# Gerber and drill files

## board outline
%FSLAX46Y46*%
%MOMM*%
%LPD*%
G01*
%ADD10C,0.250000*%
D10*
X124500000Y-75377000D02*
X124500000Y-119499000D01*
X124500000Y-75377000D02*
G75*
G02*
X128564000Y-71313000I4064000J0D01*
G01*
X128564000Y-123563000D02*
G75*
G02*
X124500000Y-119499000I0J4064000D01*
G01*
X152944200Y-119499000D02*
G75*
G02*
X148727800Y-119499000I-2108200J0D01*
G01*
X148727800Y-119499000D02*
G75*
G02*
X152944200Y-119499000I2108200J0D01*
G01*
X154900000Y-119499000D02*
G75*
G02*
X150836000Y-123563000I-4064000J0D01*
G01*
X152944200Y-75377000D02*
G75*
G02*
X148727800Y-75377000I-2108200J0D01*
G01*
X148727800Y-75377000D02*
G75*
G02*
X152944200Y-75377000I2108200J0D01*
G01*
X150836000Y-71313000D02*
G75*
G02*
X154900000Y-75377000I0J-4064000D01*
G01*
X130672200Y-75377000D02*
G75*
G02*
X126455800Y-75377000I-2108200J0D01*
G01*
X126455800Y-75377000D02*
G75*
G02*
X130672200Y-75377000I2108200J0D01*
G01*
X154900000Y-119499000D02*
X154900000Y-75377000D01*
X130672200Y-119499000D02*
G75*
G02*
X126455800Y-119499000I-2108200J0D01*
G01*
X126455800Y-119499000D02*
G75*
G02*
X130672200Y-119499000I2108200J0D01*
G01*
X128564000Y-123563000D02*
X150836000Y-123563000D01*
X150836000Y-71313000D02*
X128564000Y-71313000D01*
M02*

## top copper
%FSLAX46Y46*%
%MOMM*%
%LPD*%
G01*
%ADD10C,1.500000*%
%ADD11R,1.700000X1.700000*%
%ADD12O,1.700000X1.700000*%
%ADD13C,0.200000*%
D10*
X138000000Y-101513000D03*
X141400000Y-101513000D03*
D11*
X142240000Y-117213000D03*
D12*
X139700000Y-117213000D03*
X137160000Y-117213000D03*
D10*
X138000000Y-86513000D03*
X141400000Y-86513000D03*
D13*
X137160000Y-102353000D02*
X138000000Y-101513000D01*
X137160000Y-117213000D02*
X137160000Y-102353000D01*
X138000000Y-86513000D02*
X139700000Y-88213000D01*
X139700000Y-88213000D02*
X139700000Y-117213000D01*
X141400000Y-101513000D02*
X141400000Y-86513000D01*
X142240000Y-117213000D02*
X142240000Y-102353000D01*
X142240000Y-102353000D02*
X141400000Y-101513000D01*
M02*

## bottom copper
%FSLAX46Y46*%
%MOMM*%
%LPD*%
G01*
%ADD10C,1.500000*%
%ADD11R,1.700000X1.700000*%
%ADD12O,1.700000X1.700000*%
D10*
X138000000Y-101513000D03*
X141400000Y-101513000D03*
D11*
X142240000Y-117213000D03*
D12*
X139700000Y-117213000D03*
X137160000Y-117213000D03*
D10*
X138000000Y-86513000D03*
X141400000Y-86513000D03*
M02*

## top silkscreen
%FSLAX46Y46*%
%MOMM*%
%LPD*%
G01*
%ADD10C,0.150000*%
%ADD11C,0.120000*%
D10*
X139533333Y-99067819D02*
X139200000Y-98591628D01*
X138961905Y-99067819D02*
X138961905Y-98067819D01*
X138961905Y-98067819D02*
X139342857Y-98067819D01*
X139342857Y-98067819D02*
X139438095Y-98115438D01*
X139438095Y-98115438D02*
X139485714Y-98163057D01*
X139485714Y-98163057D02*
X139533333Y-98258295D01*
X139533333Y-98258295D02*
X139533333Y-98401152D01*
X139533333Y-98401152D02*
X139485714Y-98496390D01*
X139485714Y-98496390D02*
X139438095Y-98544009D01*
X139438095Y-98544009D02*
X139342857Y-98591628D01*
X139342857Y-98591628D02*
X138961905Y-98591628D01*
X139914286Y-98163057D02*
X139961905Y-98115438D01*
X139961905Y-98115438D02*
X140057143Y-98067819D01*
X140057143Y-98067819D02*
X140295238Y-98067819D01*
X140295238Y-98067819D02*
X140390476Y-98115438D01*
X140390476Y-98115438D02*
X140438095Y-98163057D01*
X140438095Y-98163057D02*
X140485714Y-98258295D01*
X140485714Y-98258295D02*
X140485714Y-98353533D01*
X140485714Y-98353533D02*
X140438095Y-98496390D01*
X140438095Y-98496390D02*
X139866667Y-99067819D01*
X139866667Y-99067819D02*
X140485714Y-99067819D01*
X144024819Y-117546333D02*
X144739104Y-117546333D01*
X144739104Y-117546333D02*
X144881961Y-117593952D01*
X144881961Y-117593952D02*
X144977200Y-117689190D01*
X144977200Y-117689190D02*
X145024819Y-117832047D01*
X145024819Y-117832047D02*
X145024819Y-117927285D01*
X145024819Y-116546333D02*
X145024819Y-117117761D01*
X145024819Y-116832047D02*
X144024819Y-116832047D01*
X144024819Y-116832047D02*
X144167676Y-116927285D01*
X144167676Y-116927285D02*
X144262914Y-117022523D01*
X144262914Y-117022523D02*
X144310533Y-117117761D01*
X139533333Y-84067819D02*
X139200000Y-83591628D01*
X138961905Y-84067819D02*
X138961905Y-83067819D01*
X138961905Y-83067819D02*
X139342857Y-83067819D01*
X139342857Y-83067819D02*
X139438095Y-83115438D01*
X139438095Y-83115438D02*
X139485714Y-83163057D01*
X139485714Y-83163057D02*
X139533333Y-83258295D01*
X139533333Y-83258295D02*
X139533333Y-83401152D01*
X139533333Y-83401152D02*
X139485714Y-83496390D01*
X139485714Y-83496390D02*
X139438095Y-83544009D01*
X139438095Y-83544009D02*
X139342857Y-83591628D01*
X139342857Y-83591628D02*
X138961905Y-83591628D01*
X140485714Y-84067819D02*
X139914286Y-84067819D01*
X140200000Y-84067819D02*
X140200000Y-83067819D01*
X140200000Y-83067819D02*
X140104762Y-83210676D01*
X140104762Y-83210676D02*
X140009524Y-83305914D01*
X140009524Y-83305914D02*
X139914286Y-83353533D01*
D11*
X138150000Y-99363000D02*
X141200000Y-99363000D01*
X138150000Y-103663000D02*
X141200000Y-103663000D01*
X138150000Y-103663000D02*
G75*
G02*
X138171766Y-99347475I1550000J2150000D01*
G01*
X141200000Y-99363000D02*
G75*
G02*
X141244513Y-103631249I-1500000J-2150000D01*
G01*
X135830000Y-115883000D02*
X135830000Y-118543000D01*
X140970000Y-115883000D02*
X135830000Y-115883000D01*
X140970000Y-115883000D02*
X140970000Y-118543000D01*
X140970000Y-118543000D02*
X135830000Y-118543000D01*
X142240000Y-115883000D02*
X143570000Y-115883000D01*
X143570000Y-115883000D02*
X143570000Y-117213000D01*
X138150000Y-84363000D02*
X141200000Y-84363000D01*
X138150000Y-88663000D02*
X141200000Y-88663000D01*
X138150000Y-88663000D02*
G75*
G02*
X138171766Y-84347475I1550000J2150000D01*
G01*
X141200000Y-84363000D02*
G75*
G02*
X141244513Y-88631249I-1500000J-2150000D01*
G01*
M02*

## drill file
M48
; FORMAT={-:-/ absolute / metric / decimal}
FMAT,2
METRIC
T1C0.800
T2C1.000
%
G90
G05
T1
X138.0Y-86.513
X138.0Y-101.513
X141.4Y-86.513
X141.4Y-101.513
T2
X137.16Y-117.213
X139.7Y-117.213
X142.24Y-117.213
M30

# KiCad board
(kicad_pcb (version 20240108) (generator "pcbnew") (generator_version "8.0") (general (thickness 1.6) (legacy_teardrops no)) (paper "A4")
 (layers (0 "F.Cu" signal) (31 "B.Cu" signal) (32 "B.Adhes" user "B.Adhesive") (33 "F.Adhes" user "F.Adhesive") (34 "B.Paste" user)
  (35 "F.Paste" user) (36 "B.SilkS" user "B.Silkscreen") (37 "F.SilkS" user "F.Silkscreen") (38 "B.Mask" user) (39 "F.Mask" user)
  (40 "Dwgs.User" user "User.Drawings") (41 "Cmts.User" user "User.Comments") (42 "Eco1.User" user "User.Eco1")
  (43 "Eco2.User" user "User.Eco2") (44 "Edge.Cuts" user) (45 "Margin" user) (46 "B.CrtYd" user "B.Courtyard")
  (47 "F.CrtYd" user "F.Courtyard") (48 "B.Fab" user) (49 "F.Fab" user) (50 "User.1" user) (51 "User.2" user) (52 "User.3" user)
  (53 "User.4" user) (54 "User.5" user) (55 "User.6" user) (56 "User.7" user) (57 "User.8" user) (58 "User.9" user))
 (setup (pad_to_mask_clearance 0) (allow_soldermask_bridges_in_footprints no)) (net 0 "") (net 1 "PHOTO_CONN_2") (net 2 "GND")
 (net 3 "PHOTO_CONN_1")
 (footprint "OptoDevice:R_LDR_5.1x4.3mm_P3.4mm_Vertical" (layer "F.Cu") (at 138 101.513)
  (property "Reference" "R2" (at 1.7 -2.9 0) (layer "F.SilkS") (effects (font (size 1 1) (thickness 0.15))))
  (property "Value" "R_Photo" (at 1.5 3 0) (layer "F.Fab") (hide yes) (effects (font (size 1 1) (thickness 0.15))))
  (fp_line (start 0.15 -2.15) (end 3.2 -2.15) (stroke (width 0.12) (type solid)) (layer "F.SilkS"))
  (fp_line (start 0.15 2.15) (end 3.2 2.15) (stroke (width 0.12) (type solid)) (layer "F.SilkS"))
  (fp_arc (start 0.15 2.15) (mid -0.950438 -0.013368) (end 0.171766 -2.165525) (stroke (width 0.12) (type solid)) (layer "F.SilkS"))
  (fp_arc (start 3.2 -2.15) (mid 4.321403 -0.027338) (end 3.244513 2.118249) (stroke (width 0.12) (type solid)) (layer "F.SilkS"))
  (pad "1" thru_hole circle (at 0 0) (size 1.5 1.5) (drill 0.8) (layers "*.Cu" "*.Mask") (remove_unused_layers no) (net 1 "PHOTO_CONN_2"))
  (pad "2" thru_hole circle (at 3.4 0) (size 1.5 1.5) (drill 0.8) (layers "*.Cu" "*.Mask") (remove_unused_layers no) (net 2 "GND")))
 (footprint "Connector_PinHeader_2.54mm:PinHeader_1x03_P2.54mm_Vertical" (layer "F.Cu") (at 142.24 117.213 -90)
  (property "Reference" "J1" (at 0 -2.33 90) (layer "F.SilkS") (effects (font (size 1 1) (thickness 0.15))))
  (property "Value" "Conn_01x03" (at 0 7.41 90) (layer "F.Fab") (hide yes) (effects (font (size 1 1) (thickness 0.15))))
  (fp_line (start -1.33 6.41) (end 1.33 6.41) (stroke (width 0.12) (type solid)) (layer "F.SilkS"))
  (fp_line (start -1.33 1.27) (end -1.33 6.41) (stroke (width 0.12) (type solid)) (layer "F.SilkS"))
  (fp_line (start -1.33 1.27) (end 1.33 1.27) (stroke (width 0.12) (type solid)) (layer "F.SilkS"))
  (fp_line (start 1.33 1.27) (end 1.33 6.41) (stroke (width 0.12) (type solid)) (layer "F.SilkS"))
  (fp_line (start -1.33 0) (end -1.33 -1.33) (stroke (width 0.12) (type solid)) (layer "F.SilkS"))
  (fp_line (start -1.33 -1.33) (end 0 -1.33) (stroke (width 0.12) (type solid)) (layer "F.SilkS"))
  (pad "1" thru_hole rect (at 0 0 270) (size 1.7 1.7) (drill 1) (layers "*.Cu" "*.Mask") (remove_unused_layers no) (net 2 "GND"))
  (pad "2" thru_hole oval (at 0 2.54 270) (size 1.7 1.7) (drill 1) (layers "*.Cu" "*.Mask") (remove_unused_layers no) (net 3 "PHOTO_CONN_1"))
  (pad "3" thru_hole oval (at 0 5.08 270) (size 1.7 1.7) (drill 1) (layers "*.Cu" "*.Mask") (remove_unused_layers no) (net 1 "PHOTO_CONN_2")))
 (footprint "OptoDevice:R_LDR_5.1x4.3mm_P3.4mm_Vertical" (layer "F.Cu") (at 138 86.513)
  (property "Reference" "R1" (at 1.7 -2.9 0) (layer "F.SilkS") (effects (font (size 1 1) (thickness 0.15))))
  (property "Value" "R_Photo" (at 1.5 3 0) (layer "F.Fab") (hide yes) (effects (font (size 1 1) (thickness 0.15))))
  (fp_line (start 0.15 -2.15) (end 3.2 -2.15) (stroke (width 0.12) (type solid)) (layer "F.SilkS"))
  (fp_line (start 0.15 2.15) (end 3.2 2.15) (stroke (width 0.12) (type solid)) (layer "F.SilkS"))
  (fp_arc (start 0.15 2.15) (mid -0.950438 -0.013368) (end 0.171766 -2.165525) (stroke (width 0.12) (type solid)) (layer "F.SilkS"))
  (fp_arc (start 3.2 -2.15) (mid 4.321403 -0.027338) (end 3.244513 2.118249) (stroke (width 0.12) (type solid)) (layer "F.SilkS"))
  (pad "1" thru_hole circle (at 0 0) (size 1.5 1.5) (drill 0.8) (layers "*.Cu" "*.Mask") (remove_unused_layers no) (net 3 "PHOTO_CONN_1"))
  (pad "2" thru_hole circle (at 3.4 0) (size 1.5 1.5) (drill 0.8) (layers "*.Cu" "*.Mask") (remove_unused_layers no) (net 2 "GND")))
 (gr_line (start 124.5 75.377) (end 124.5 119.499) (locked yes) (stroke (width 0.25) (type default)) (layer "Edge.Cuts"))
 (gr_arc (start 124.5 75.377) (mid 125.690318 72.503318) (end 128.564 71.313) (locked yes) (stroke (width 0.25) (type default))
  (layer "Edge.Cuts"))
 (gr_arc (start 128.564 123.563) (mid 125.690318 122.372682) (end 124.5 119.499) (locked yes) (stroke (width 0.25) (type default))
  (layer "Edge.Cuts"))
 (gr_circle (center 150.836 119.499) (end 152.9442 119.499) (locked yes) (stroke (width 0.25) (type default)) (fill none)
  (layer "Edge.Cuts"))
 (gr_arc (start 154.9 119.499) (mid 153.709682 122.372682) (end 150.836 123.563) (locked yes) (stroke (width 0.25) (type default))
  (layer "Edge.Cuts"))
 (gr_circle (center 150.836 75.377) (end 152.9442 75.377) (locked yes) (stroke (width 0.25) (type default)) (fill none) (layer "Edge.Cuts"))
 (gr_arc (start 150.836 71.313) (mid 153.709682 72.503318) (end 154.9 75.377) (locked yes) (stroke (width 0.25) (type default))
  (layer "Edge.Cuts"))
 (gr_circle (center 128.564 75.377) (end 130.6722 75.377) (locked yes) (stroke (width 0.25) (type default)) (fill none) (layer "Edge.Cuts"))
 (gr_line (start 154.9 119.499) (end 154.9 75.377) (locked yes) (stroke (width 0.25) (type default)) (layer "Edge.Cuts"))
 (gr_circle (center 128.564 119.499) (end 130.6722 119.499) (locked yes) (stroke (width 0.25) (type default)) (fill none)
  (layer "Edge.Cuts"))
 (gr_line (start 128.564 123.563) (end 150.836 123.563) (locked yes) (stroke (width 0.25) (type default)) (layer "Edge.Cuts"))
 (gr_line (start 150.836 71.313) (end 128.564 71.313) (locked yes) (stroke (width 0.25) (type default)) (layer "Edge.Cuts"))
 (segment (start 137.16 102.353) (end 138 101.513) (width 0.2) (layer "F.Cu") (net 1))
 (segment (start 137.16 117.213) (end 137.16 102.353) (width 0.2) (layer "F.Cu") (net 1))
 (segment (start 138 86.513) (end 139.7 88.213) (width 0.2) (layer "F.Cu") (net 3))
 (segment (start 139.7 88.213) (end 139.7 117.213) (width 0.2) (layer "F.Cu") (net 3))
 (segment (start 141.4 101.513) (end 141.4 86.513) (width 0.2) (layer "F.Cu") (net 2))
 (segment (start 142.24 117.213) (end 142.24 102.353) (width 0.2) (layer "F.Cu") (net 2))
 (segment (start 142.24 102.353) (end 141.4 101.513) (width 0.2) (layer "F.Cu") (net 2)))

